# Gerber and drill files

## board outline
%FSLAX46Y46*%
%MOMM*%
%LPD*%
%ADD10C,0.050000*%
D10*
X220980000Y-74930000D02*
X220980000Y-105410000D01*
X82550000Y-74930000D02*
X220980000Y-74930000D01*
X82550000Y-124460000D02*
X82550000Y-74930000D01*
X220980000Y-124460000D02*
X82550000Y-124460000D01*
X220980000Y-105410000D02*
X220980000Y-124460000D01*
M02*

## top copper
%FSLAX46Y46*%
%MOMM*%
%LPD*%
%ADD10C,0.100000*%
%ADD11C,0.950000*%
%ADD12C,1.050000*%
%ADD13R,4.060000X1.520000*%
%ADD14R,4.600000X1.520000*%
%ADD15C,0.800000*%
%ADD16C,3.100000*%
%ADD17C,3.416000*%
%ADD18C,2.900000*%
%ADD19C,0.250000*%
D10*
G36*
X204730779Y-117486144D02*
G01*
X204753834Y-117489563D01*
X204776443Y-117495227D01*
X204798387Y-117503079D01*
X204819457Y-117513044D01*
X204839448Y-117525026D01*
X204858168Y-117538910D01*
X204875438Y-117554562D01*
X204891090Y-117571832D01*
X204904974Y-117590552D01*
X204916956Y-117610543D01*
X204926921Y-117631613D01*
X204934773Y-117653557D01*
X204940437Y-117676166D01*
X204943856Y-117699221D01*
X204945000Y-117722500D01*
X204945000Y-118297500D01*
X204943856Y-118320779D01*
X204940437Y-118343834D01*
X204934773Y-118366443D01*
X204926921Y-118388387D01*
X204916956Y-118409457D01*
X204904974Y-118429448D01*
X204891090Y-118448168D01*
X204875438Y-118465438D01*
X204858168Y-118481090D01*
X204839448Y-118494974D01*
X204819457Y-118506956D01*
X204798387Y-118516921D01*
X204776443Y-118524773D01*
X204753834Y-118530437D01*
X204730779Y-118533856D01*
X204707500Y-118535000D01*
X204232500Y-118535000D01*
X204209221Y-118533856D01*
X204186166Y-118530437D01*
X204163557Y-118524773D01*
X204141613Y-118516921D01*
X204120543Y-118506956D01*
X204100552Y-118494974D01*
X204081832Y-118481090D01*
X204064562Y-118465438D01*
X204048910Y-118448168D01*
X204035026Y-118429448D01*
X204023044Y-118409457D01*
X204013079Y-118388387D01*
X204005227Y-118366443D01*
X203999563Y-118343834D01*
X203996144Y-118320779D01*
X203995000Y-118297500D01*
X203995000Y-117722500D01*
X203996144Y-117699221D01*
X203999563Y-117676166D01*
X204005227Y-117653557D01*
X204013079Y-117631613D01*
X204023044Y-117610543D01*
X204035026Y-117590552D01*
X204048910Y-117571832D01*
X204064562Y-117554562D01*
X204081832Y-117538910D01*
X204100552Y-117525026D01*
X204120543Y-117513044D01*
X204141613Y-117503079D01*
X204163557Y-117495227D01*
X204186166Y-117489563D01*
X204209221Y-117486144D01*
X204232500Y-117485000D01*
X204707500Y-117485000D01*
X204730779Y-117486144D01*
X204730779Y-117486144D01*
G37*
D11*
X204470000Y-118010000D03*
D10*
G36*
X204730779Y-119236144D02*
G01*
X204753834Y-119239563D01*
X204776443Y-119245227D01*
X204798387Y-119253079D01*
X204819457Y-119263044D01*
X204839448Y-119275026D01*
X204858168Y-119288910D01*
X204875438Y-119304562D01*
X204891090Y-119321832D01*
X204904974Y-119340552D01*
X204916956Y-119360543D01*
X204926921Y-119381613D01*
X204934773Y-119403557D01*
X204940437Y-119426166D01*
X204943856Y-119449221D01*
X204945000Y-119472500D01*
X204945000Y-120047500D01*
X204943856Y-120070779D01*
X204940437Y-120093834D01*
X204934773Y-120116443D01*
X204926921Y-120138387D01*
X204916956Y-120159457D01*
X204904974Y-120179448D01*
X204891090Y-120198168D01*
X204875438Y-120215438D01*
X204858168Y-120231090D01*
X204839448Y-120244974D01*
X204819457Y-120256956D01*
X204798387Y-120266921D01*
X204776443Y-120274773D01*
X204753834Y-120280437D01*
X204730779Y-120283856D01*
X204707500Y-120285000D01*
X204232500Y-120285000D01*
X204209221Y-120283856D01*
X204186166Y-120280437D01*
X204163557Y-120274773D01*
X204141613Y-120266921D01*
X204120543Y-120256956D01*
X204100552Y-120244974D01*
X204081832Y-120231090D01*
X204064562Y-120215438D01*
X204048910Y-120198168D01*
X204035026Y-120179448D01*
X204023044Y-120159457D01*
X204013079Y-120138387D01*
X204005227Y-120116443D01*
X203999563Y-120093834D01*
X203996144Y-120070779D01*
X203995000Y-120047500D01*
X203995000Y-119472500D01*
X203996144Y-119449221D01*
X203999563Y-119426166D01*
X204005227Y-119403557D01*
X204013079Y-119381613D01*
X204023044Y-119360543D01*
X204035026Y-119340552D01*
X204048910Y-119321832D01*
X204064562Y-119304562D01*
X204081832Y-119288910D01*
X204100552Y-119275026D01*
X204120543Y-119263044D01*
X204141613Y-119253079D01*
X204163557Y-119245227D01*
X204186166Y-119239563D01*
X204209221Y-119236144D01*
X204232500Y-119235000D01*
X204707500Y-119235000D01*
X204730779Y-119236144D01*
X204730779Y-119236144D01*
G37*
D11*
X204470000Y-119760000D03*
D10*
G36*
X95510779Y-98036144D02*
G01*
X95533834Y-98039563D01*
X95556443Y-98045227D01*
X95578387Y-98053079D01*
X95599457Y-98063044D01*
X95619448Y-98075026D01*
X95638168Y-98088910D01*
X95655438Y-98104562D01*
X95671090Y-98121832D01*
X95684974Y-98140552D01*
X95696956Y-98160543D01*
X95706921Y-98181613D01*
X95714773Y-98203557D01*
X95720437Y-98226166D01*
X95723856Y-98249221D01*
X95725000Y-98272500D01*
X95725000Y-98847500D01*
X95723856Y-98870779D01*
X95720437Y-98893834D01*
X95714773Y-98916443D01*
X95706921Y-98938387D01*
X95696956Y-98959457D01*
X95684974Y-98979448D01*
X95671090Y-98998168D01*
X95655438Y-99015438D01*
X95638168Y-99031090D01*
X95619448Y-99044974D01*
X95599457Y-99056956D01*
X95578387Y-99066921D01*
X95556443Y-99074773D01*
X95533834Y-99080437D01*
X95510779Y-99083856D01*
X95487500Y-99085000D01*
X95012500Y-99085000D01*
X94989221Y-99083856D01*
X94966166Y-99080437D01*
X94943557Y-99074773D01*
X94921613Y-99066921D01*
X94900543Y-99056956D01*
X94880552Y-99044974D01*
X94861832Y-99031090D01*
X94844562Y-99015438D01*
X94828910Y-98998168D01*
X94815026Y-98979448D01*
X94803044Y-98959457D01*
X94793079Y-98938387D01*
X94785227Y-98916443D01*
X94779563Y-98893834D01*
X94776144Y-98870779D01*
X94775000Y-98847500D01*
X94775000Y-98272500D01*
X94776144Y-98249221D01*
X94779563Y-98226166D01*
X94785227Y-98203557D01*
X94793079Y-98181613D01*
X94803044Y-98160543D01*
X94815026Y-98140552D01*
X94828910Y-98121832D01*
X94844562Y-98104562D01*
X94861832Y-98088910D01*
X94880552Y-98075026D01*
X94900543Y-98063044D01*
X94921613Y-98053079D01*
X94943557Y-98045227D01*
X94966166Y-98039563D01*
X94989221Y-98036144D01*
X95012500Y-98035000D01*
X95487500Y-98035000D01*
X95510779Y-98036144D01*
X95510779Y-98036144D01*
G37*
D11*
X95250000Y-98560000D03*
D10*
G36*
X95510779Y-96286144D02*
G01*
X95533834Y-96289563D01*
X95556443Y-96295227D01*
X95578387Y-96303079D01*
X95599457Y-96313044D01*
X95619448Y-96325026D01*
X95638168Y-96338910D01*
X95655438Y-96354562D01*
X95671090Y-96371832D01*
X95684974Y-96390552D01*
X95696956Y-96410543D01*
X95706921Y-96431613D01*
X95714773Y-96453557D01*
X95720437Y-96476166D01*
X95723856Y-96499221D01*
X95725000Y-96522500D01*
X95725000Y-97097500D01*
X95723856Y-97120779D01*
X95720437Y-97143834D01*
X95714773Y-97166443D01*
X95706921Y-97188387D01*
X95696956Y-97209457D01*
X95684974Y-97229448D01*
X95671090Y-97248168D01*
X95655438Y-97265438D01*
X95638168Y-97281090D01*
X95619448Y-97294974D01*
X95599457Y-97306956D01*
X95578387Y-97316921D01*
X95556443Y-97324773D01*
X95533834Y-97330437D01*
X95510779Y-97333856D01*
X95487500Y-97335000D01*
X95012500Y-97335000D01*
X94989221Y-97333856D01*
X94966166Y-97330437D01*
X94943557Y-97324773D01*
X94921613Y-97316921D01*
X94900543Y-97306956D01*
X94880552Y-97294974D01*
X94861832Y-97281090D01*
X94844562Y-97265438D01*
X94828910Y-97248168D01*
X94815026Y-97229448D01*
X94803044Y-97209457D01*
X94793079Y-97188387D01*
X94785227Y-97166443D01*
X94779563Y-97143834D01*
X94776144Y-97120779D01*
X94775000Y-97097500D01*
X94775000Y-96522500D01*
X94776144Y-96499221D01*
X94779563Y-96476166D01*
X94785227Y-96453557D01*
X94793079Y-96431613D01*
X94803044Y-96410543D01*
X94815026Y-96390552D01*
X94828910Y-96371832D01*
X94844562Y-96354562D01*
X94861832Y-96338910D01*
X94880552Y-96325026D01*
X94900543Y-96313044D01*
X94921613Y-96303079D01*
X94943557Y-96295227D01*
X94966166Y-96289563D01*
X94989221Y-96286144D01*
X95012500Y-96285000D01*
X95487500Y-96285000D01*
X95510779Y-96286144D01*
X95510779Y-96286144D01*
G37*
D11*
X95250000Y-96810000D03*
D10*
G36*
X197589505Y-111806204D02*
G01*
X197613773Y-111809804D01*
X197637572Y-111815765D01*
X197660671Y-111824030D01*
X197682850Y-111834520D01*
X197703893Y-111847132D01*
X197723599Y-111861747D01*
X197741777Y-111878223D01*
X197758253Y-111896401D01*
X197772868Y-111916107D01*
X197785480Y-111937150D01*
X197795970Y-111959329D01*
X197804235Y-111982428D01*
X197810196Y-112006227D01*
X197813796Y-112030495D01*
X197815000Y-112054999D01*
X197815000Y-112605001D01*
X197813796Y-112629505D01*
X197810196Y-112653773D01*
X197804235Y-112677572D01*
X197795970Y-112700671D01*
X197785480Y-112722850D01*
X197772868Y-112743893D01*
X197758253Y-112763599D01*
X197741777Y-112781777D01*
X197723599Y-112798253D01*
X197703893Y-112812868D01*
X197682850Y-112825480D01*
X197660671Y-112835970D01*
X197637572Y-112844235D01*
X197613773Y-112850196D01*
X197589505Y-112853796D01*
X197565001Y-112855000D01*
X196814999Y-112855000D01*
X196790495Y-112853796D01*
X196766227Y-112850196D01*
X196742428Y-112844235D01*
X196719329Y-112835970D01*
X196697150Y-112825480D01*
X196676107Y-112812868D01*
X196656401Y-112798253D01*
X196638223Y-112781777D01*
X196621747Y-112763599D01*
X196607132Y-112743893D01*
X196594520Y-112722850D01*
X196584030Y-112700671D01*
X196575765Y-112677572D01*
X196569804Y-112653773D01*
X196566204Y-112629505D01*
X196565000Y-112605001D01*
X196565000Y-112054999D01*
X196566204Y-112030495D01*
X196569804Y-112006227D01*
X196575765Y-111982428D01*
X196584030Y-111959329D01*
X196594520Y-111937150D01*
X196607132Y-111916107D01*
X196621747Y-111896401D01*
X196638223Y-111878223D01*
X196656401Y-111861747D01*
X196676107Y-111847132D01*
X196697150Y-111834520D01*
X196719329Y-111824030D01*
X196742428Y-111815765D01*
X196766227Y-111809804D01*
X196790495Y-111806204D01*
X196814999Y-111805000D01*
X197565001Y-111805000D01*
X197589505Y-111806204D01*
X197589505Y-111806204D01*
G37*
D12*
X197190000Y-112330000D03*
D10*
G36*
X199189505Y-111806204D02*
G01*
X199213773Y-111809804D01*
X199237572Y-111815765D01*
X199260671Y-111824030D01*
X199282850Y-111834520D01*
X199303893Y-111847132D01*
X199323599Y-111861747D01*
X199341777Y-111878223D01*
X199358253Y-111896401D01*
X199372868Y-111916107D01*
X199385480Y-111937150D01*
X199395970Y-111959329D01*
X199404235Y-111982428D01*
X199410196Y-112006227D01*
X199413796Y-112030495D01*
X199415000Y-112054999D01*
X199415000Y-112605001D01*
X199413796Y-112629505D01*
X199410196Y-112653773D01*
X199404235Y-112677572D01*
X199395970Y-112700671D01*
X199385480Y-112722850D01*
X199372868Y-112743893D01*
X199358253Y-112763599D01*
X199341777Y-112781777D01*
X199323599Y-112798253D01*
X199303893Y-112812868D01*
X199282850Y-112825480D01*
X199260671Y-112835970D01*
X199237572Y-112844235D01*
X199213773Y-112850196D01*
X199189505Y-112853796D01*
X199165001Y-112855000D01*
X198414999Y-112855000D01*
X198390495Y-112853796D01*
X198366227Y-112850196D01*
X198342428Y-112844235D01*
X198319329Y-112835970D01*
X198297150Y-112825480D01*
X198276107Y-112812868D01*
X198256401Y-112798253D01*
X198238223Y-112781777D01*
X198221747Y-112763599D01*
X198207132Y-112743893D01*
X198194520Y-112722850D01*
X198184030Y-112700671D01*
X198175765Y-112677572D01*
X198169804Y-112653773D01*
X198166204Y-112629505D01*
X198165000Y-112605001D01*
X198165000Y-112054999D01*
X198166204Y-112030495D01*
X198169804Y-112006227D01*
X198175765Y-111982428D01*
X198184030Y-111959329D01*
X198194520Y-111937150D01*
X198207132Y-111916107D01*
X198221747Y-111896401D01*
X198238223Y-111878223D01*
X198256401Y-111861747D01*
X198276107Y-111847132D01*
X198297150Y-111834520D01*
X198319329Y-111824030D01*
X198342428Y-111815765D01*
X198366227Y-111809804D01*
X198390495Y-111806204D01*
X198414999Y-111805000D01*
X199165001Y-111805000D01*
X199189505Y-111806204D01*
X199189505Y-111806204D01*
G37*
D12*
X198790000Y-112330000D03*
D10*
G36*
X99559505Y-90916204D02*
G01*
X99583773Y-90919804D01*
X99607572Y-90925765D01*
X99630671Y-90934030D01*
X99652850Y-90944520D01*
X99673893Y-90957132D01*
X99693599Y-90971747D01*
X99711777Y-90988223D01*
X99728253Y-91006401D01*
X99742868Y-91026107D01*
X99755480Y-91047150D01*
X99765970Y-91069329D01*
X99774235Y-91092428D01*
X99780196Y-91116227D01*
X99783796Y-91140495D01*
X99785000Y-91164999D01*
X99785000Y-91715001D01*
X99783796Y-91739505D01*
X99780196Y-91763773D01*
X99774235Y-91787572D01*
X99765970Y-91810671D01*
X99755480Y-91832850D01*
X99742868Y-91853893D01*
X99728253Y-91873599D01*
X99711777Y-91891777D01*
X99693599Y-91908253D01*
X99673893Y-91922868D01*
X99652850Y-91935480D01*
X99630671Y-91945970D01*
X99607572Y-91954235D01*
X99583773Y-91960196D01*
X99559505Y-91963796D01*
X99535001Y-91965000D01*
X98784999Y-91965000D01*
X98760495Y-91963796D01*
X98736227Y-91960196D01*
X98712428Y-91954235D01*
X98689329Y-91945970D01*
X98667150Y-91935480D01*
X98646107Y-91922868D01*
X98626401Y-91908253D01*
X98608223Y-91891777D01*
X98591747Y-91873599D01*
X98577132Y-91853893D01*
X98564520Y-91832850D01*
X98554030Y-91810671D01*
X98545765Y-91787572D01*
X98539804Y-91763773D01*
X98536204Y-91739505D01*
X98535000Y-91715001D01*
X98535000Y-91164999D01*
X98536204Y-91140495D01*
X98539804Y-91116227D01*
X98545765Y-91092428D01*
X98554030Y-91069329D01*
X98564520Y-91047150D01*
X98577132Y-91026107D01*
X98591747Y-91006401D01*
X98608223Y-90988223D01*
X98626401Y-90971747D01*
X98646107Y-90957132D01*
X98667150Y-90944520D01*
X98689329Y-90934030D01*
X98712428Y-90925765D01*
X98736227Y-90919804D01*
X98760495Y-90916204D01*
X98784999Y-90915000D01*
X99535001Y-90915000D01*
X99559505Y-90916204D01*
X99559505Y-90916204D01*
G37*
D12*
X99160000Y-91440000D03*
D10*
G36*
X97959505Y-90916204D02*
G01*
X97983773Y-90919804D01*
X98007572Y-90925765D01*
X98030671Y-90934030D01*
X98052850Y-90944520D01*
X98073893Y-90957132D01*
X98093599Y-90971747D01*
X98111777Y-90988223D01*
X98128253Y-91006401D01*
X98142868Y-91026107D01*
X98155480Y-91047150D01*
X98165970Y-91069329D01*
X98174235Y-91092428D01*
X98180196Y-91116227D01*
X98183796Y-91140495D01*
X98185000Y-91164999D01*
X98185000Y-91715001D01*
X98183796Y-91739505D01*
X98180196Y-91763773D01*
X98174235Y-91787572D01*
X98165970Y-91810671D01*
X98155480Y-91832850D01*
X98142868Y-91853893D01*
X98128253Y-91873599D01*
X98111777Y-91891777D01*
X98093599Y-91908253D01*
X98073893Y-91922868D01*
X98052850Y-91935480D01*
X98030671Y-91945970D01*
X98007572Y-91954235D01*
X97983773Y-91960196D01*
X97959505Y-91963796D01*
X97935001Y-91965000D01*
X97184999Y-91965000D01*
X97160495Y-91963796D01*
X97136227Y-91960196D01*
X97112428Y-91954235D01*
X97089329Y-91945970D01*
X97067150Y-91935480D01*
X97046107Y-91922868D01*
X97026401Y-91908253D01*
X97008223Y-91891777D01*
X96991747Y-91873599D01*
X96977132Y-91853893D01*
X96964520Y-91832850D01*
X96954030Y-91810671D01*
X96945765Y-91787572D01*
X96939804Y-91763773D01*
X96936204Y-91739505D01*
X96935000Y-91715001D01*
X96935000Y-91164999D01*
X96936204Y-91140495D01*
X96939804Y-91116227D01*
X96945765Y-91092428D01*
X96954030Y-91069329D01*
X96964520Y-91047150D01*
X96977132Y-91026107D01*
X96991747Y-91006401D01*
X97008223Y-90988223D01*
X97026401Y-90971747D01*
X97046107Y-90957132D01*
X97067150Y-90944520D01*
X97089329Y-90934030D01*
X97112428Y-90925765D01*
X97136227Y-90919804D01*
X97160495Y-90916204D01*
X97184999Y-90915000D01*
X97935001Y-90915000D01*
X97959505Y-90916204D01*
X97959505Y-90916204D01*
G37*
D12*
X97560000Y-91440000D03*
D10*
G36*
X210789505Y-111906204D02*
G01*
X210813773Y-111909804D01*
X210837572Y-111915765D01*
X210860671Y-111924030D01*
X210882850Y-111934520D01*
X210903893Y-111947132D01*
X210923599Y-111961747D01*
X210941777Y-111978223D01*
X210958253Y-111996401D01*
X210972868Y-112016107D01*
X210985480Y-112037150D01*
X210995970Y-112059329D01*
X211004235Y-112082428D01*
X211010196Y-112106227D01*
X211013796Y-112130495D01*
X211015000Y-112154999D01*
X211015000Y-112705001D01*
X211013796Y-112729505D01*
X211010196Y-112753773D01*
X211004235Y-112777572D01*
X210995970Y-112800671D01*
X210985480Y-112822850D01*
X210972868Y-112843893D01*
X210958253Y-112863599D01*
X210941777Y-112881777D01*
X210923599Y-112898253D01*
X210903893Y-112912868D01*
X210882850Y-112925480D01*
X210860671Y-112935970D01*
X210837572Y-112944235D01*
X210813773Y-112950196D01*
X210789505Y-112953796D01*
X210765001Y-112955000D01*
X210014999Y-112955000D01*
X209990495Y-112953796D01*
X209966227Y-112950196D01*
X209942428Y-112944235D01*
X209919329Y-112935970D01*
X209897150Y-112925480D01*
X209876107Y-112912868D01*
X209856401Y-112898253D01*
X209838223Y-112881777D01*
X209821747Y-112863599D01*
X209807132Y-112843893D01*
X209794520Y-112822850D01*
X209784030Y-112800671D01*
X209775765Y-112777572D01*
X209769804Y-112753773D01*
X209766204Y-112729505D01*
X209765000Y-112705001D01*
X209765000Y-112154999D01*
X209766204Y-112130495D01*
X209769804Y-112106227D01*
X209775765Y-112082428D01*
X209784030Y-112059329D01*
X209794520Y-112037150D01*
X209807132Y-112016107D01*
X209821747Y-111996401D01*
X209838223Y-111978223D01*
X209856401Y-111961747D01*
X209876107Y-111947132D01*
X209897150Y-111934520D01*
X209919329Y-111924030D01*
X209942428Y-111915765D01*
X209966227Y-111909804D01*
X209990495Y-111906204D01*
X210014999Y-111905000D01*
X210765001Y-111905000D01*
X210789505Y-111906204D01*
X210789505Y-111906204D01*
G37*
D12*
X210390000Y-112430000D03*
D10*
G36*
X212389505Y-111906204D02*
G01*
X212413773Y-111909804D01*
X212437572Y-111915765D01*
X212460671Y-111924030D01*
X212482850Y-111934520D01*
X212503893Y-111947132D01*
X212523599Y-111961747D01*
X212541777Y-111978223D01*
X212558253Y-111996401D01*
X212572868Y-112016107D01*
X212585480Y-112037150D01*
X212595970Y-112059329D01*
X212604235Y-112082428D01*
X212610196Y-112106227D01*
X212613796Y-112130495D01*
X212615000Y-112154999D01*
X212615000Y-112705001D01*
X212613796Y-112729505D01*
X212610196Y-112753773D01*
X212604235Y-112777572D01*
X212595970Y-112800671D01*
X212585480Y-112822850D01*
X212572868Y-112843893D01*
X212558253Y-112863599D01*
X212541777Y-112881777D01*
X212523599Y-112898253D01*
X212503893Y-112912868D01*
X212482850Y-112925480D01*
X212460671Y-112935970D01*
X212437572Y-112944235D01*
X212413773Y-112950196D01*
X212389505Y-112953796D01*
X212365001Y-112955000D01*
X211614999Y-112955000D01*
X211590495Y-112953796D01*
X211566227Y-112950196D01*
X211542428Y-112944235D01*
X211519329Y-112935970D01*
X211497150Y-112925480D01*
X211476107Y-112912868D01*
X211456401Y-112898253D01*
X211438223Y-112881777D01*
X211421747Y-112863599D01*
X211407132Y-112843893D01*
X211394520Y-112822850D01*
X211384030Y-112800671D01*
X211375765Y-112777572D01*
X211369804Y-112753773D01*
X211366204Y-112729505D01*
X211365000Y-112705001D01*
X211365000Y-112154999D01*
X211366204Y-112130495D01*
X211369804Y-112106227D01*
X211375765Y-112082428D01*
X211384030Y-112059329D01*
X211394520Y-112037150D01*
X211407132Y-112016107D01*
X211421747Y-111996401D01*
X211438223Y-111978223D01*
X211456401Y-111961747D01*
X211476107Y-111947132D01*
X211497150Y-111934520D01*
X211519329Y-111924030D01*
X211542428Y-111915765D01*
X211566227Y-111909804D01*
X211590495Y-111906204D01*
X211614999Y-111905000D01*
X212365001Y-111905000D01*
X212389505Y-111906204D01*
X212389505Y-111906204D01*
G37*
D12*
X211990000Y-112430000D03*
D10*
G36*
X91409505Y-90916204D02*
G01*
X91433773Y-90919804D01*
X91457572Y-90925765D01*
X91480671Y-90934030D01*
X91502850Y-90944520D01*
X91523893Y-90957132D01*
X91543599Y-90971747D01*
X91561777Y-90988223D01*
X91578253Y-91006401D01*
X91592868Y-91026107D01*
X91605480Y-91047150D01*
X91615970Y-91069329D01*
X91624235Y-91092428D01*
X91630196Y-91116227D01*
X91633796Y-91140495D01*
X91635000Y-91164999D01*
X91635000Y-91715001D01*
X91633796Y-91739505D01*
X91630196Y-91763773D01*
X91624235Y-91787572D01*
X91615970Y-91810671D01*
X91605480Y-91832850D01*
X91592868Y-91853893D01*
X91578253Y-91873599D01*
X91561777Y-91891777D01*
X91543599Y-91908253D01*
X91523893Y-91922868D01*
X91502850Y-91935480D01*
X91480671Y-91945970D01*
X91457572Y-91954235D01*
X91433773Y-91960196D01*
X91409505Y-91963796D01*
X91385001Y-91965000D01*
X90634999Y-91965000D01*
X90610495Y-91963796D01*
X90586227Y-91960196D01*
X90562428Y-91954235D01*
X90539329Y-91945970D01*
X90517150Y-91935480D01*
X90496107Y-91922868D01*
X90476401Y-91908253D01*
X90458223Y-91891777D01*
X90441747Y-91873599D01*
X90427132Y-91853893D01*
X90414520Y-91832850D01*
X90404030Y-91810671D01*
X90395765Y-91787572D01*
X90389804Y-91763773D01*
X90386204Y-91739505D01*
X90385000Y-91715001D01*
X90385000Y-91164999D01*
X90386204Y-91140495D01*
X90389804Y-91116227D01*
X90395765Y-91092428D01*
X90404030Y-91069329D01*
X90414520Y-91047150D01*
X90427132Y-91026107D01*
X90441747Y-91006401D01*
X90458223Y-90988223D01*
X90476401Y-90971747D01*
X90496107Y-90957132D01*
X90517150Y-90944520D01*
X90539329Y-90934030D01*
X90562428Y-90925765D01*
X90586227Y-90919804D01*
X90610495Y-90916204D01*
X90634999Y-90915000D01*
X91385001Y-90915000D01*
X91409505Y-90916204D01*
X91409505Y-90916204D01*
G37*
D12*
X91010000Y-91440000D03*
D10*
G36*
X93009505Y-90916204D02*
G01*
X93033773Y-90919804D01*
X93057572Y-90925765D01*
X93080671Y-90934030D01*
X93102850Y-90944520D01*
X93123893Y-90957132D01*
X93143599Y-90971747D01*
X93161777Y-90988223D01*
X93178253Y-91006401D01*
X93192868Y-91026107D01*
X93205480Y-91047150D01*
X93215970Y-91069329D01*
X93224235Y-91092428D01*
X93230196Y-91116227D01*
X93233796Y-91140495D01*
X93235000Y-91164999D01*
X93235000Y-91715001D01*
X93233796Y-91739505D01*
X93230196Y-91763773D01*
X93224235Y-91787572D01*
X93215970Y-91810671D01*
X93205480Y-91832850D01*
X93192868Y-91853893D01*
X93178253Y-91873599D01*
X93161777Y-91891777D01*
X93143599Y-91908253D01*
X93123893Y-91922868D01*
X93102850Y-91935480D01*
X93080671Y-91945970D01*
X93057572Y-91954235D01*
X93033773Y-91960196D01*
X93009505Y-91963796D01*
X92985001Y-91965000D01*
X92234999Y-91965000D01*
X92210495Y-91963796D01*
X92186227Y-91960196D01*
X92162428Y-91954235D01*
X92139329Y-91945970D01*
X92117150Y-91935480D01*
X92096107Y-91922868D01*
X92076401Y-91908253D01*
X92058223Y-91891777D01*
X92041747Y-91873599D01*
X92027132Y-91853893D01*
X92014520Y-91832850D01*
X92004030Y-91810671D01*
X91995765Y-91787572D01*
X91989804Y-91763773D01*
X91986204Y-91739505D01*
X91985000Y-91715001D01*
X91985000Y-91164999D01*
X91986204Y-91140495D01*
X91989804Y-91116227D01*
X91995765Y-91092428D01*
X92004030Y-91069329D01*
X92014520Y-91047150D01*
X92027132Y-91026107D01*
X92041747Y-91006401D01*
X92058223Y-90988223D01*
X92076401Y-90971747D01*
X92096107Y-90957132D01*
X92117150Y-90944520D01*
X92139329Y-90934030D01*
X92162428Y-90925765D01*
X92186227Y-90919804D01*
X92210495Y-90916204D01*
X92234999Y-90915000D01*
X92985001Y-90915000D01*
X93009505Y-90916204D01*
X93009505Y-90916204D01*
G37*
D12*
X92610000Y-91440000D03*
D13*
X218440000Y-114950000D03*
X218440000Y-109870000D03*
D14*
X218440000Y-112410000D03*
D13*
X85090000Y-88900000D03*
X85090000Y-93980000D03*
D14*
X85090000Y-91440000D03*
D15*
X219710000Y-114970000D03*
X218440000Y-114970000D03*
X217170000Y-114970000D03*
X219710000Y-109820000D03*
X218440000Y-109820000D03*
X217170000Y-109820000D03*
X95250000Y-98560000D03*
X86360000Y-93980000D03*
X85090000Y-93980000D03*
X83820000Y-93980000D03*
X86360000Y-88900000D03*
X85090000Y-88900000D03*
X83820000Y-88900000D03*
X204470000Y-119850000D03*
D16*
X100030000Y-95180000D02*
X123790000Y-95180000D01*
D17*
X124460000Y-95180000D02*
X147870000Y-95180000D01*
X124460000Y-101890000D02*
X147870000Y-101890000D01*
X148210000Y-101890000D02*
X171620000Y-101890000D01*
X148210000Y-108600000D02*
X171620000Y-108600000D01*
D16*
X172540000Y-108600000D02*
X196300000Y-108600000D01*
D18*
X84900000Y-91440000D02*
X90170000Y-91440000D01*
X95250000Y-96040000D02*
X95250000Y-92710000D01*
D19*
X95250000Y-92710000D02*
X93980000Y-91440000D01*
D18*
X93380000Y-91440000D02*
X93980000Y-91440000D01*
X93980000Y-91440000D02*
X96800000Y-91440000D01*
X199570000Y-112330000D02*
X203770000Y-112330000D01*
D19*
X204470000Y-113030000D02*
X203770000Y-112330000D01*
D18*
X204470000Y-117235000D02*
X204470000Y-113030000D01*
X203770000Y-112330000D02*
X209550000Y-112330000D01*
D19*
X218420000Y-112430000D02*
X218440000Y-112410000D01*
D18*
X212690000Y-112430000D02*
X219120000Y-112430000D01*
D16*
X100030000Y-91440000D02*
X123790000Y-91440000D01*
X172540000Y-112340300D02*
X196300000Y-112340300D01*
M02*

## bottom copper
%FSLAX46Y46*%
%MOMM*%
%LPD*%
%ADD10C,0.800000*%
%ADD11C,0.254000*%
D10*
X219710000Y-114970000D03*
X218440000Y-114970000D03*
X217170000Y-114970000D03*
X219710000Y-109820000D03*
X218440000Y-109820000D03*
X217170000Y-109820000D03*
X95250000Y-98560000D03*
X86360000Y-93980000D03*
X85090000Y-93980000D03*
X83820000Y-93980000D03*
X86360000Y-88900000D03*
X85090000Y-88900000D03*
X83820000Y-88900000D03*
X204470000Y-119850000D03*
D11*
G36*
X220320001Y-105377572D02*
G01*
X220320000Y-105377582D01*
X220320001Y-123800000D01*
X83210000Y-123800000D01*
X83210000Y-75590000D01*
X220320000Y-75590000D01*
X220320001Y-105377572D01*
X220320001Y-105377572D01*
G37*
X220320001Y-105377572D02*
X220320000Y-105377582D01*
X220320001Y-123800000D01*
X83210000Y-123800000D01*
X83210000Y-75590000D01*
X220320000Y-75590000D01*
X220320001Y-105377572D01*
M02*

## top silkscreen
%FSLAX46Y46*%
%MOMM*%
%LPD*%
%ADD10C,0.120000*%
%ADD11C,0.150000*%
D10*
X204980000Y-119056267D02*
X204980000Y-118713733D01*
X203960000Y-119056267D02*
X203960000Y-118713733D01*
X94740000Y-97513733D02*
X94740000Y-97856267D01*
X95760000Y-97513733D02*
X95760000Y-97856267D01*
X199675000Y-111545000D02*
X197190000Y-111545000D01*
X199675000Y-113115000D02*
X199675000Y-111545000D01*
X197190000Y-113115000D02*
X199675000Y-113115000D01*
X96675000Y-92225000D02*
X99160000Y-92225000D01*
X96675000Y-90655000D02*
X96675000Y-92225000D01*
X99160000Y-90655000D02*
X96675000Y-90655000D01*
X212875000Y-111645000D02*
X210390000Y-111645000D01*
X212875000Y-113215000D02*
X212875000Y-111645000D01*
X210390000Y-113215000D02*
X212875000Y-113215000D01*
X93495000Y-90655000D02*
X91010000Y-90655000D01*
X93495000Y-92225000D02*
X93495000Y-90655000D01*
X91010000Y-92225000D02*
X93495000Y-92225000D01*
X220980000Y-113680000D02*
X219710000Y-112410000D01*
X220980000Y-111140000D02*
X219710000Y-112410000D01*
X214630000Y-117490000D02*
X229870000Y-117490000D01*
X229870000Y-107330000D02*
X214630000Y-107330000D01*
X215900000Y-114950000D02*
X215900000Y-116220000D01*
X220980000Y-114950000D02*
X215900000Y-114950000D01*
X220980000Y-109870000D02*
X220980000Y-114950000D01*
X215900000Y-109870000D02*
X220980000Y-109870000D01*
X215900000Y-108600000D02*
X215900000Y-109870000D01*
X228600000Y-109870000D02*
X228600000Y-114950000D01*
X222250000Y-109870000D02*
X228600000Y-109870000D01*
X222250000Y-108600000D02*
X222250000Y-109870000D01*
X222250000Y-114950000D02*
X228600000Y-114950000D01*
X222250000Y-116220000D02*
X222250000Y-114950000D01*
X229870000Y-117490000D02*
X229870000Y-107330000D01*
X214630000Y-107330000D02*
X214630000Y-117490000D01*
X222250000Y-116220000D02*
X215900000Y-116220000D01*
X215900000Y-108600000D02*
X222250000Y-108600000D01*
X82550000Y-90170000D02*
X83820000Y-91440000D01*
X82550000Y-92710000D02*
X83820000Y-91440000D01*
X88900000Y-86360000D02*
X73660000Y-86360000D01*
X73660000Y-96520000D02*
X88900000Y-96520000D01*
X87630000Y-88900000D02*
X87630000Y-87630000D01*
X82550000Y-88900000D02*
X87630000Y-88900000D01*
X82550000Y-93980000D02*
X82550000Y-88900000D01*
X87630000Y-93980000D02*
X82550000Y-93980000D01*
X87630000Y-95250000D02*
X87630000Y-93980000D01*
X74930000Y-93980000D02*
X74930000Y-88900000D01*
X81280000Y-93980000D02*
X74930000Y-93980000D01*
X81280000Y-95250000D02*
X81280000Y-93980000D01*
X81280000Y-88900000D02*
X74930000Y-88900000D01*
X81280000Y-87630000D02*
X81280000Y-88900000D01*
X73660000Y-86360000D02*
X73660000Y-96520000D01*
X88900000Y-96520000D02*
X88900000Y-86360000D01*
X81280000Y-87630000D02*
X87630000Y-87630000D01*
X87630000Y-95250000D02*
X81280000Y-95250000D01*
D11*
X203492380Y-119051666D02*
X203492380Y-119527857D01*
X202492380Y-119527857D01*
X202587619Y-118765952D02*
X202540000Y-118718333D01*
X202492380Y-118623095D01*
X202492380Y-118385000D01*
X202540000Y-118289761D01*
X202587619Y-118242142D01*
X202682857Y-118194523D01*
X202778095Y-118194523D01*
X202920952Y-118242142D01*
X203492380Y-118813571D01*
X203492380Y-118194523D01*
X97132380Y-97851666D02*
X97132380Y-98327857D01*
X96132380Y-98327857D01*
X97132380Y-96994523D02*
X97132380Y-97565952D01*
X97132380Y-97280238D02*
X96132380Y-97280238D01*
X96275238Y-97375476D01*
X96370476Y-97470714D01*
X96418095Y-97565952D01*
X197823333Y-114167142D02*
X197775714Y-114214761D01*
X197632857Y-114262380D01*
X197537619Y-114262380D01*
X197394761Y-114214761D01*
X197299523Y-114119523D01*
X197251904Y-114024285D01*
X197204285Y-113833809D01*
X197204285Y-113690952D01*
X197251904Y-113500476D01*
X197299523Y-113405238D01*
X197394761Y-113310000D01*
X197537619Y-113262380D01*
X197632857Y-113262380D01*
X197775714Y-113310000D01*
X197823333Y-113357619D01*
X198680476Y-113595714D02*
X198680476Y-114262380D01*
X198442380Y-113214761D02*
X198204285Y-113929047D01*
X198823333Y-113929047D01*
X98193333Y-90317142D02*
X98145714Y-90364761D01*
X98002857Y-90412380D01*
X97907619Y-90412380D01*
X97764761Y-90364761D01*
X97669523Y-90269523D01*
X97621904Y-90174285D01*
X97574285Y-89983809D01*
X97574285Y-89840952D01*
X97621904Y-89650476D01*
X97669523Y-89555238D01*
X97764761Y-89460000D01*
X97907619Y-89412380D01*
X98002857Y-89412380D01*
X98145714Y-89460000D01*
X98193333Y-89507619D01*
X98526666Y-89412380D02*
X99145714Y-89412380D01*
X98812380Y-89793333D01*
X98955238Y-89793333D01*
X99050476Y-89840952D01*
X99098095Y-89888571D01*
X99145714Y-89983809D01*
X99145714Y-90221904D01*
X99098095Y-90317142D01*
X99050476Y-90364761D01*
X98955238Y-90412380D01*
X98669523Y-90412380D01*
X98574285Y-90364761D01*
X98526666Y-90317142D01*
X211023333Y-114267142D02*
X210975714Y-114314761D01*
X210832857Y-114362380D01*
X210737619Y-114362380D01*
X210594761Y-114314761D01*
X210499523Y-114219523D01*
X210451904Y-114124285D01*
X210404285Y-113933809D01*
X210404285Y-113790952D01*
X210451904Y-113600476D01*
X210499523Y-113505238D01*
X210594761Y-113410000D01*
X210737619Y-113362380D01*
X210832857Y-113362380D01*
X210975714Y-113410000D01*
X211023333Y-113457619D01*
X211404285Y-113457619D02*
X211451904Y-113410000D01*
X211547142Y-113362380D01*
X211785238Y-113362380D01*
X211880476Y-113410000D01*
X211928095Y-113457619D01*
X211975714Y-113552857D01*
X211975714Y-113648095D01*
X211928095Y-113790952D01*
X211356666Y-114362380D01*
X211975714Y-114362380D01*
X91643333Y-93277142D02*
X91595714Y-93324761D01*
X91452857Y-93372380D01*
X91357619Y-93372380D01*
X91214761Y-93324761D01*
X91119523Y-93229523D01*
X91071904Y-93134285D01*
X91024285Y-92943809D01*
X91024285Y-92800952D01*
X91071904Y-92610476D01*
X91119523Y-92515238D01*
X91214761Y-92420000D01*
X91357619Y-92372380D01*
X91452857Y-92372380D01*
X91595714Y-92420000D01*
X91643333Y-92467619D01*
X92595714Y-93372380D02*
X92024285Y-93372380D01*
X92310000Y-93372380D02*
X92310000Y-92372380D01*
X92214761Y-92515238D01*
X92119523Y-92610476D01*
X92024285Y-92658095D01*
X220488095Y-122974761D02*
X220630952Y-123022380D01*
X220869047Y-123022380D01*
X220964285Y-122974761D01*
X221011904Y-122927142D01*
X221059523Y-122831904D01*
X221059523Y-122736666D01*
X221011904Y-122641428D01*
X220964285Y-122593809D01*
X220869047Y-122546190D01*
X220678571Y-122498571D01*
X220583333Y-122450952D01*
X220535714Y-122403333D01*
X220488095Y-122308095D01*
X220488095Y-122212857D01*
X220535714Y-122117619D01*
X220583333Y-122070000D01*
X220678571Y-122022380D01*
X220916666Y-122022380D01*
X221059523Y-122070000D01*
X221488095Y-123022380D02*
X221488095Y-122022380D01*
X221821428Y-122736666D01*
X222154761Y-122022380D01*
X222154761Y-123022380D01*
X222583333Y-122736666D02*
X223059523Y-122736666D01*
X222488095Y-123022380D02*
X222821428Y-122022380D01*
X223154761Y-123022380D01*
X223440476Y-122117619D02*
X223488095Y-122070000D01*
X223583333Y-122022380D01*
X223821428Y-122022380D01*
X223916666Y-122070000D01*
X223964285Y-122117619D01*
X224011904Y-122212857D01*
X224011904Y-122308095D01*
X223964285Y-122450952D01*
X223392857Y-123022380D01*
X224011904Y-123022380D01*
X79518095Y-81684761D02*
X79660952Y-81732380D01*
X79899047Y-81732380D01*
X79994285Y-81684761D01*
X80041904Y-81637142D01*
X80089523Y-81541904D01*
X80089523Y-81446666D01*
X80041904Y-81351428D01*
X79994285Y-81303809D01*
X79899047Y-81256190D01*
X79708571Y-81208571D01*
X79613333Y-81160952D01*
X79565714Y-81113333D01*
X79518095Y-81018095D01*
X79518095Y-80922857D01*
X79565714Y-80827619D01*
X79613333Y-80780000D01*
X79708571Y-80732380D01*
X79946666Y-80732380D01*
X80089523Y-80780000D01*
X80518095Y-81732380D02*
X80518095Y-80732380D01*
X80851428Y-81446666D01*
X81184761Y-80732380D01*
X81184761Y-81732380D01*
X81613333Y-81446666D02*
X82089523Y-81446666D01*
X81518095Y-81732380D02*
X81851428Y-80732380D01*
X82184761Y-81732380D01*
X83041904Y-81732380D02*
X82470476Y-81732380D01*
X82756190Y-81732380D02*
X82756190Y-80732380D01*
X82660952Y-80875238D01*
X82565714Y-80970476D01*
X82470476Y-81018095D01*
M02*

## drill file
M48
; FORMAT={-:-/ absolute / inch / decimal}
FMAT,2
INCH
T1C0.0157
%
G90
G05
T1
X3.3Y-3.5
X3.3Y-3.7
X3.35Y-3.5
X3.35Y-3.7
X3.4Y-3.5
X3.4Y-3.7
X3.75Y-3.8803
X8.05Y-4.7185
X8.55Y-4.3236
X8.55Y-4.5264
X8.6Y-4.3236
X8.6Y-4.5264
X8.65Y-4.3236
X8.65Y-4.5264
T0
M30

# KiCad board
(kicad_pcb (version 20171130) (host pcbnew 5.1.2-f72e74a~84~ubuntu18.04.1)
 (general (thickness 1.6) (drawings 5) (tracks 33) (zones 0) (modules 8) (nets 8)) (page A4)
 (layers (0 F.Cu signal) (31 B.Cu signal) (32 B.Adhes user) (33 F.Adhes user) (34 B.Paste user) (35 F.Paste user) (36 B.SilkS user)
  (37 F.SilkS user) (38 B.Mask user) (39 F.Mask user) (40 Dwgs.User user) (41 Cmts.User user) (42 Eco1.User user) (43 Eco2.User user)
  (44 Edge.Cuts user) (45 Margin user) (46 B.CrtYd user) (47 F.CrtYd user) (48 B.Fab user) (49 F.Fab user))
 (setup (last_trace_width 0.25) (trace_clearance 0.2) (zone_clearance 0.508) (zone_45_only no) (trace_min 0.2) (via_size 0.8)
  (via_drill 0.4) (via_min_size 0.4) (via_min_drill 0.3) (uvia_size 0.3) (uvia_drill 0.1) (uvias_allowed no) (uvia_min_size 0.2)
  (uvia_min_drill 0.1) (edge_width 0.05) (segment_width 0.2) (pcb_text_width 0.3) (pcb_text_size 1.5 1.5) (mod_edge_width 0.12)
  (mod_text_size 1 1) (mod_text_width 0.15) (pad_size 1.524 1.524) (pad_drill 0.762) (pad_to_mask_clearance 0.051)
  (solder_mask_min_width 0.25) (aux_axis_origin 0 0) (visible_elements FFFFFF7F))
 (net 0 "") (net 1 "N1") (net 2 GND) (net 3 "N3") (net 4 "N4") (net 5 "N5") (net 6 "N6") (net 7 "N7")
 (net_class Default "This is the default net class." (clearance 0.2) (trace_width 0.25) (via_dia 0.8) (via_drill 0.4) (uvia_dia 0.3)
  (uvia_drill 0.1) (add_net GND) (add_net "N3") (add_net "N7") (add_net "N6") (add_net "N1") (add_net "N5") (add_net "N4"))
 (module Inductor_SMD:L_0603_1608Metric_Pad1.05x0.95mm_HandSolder (layer F.Cu) (at 204.47 118.885 90)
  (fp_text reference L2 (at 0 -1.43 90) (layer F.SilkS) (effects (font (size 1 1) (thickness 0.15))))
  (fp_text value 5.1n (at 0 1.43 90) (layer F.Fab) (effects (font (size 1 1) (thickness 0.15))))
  (fp_line (start -0.171267 0.51) (end 0.171267 0.51) (layer F.SilkS) (width 0.12))
  (fp_line (start -0.171267 -0.51) (end 0.171267 -0.51) (layer F.SilkS) (width 0.12))
  (pad 2 smd roundrect (at 0.875 0 90) (size 1.05 0.95) (layers F.Cu F.Paste F.Mask) (roundrect_rratio 0.25) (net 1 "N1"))
  (pad 1 smd roundrect (at -0.875 0 90) (size 1.05 0.95) (layers F.Cu F.Paste F.Mask) (roundrect_rratio 0.25) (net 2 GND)))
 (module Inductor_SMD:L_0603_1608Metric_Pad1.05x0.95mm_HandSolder (layer F.Cu) (at 95.25 97.685 270)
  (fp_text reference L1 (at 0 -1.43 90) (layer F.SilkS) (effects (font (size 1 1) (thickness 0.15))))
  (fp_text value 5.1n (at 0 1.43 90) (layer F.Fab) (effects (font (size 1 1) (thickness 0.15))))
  (fp_line (start -0.171267 0.51) (end 0.171267 0.51) (layer F.SilkS) (width 0.12))
  (fp_line (start -0.171267 -0.51) (end 0.171267 -0.51) (layer F.SilkS) (width 0.12))
  (pad 2 smd roundrect (at 0.875 0 270) (size 1.05 0.95) (layers F.Cu F.Paste F.Mask) (roundrect_rratio 0.25) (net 2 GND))
  (pad 1 smd roundrect (at -0.875 0 270) (size 1.05 0.95) (layers F.Cu F.Paste F.Mask) (roundrect_rratio 0.25) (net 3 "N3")))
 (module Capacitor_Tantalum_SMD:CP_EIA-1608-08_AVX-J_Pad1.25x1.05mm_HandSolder (layer F.Cu) (at 197.99 112.33 180)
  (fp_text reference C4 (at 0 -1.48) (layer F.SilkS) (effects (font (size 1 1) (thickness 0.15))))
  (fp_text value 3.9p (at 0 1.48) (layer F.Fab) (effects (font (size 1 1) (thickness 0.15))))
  (fp_line (start -1.685 0.785) (end 0.8 0.785) (layer F.SilkS) (width 0.12))
  (fp_line (start -1.685 -0.785) (end -1.685 0.785) (layer F.SilkS) (width 0.12))
  (fp_line (start 0.8 -0.785) (end -1.685 -0.785) (layer F.SilkS) (width 0.12))
  (pad 2 smd roundrect (at 0.8 0 180) (size 1.25 1.05) (layers F.Cu F.Paste F.Mask) (roundrect_rratio 0.238095) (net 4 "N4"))
  (pad 1 smd roundrect (at -0.8 0 180) (size 1.25 1.05) (layers F.Cu F.Paste F.Mask) (roundrect_rratio 0.238095) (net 1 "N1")))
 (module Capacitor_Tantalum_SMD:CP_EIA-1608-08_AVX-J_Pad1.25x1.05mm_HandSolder (layer F.Cu) (at 98.36 91.44)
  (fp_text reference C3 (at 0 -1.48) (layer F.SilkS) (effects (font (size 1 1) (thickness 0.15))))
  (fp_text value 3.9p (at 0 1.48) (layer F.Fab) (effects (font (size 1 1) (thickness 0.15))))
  (fp_line (start -1.685 0.785) (end 0.8 0.785) (layer F.SilkS) (width 0.12))
  (fp_line (start -1.685 -0.785) (end -1.685 0.785) (layer F.SilkS) (width 0.12))
  (fp_line (start 0.8 -0.785) (end -1.685 -0.785) (layer F.SilkS) (width 0.12))
  (pad 2 smd roundrect (at 0.8 0) (size 1.25 1.05) (layers F.Cu F.Paste F.Mask) (roundrect_rratio 0.238095) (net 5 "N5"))
  (pad 1 smd roundrect (at -0.8 0) (size 1.25 1.05) (layers F.Cu F.Paste F.Mask) (roundrect_rratio 0.238095) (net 3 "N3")))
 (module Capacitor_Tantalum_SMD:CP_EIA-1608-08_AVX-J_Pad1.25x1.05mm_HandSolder (layer F.Cu) (at 211.19 112.43 180)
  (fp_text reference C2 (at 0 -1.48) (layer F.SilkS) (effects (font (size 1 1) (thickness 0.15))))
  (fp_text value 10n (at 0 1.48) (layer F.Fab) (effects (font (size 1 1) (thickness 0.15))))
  (fp_line (start -1.685 0.785) (end 0.8 0.785) (layer F.SilkS) (width 0.12))
  (fp_line (start -1.685 -0.785) (end -1.685 0.785) (layer F.SilkS) (width 0.12))
  (fp_line (start 0.8 -0.785) (end -1.685 -0.785) (layer F.SilkS) (width 0.12))
  (pad 2 smd roundrect (at 0.8 0 180) (size 1.25 1.05) (layers F.Cu F.Paste F.Mask) (roundrect_rratio 0.238095) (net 1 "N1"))
  (pad 1 smd roundrect (at -0.8 0 180) (size 1.25 1.05) (layers F.Cu F.Paste F.Mask) (roundrect_rratio 0.238095) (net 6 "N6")))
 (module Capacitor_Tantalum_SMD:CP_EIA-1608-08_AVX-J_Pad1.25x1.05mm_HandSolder (layer F.Cu) (at 91.81 91.44 180)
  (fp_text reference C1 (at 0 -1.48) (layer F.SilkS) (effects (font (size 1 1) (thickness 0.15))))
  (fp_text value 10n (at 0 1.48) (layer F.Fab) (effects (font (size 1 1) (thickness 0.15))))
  (fp_line (start -1.685 0.785) (end 0.8 0.785) (layer F.SilkS) (width 0.12))
  (fp_line (start -1.685 -0.785) (end -1.685 0.785) (layer F.SilkS) (width 0.12))
  (fp_line (start 0.8 -0.785) (end -1.685 -0.785) (layer F.SilkS) (width 0.12))
  (pad 2 smd roundrect (at 0.8 0 180) (size 1.25 1.05) (layers F.Cu F.Paste F.Mask) (roundrect_rratio 0.238095) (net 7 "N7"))
  (pad 1 smd roundrect (at -0.8 0 180) (size 1.25 1.05) (layers F.Cu F.Paste F.Mask) (roundrect_rratio 0.238095) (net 3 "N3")))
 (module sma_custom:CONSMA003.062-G (layer F.Cu) (at 222.25 114.95)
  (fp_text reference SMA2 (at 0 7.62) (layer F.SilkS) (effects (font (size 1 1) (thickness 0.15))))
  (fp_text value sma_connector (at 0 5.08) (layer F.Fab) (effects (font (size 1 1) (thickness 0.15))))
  (fp_line (start -1.27 -1.27) (end -2.54 -2.54) (layer F.SilkS) (width 0.12))
  (fp_line (start -1.27 -3.81) (end -2.54 -2.54) (layer F.SilkS) (width 0.12))
  (fp_line (start -7.62 2.54) (end 7.62 2.54) (layer F.SilkS) (width 0.12))
  (fp_line (start 7.62 -7.62) (end -7.62 -7.62) (layer F.SilkS) (width 0.12))
  (fp_line (start -6.35 0) (end -6.35 1.27) (layer F.SilkS) (width 0.12))
  (fp_line (start -1.27 0) (end -6.35 0) (layer F.SilkS) (width 0.12))
  (fp_line (start -1.27 -5.08) (end -1.27 0) (layer F.SilkS) (width 0.12))
  (fp_line (start -6.35 -5.08) (end -1.27 -5.08) (layer F.SilkS) (width 0.12))
  (fp_line (start -6.35 -6.35) (end -6.35 -5.08) (layer F.SilkS) (width 0.12))
  (fp_line (start 6.35 -5.08) (end 6.35 0) (layer F.SilkS) (width 0.12))
  (fp_line (start 0 -5.08) (end 6.35 -5.08) (layer F.SilkS) (width 0.12))
  (fp_line (start 0 -6.35) (end 0 -5.08) (layer F.SilkS) (width 0.12))
  (fp_line (start 0 0) (end 6.35 0) (layer F.SilkS) (width 0.12))
  (fp_line (start 0 1.27) (end 0 0) (layer F.SilkS) (width 0.12))
  (fp_line (start 7.62 2.54) (end 7.62 -7.62) (layer F.SilkS) (width 0.12))
  (fp_line (start -7.62 -7.62) (end -7.62 2.54) (layer F.SilkS) (width 0.12))
  (fp_line (start 0 1.27) (end -6.35 1.27) (layer F.SilkS) (width 0.12))
  (fp_line (start -6.35 -6.35) (end 0 -6.35) (layer F.SilkS) (width 0.12))
  (pad 3 smd rect (at -3.81 0) (size 4.06 1.52) (layers F.Cu F.Paste F.Mask) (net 2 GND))
  (pad 2 smd rect (at -3.81 -5.08) (size 4.06 1.52) (layers F.Cu F.Paste F.Mask) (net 2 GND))
  (pad 1 smd rect (at -3.81 -2.54) (size 4.6 1.52) (layers F.Cu F.Paste F.Mask) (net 6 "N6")))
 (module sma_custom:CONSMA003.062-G (layer F.Cu) (at 81.28 88.9 180)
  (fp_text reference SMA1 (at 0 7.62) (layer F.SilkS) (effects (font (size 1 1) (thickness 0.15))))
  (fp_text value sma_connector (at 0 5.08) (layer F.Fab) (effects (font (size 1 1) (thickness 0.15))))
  (fp_line (start -1.27 -1.27) (end -2.54 -2.54) (layer F.SilkS) (width 0.12))
  (fp_line (start -1.27 -3.81) (end -2.54 -2.54) (layer F.SilkS) (width 0.12))
  (fp_line (start -7.62 2.54) (end 7.62 2.54) (layer F.SilkS) (width 0.12))
  (fp_line (start 7.62 -7.62) (end -7.62 -7.62) (layer F.SilkS) (width 0.12))
  (fp_line (start -6.35 0) (end -6.35 1.27) (layer F.SilkS) (width 0.12))
  (fp_line (start -1.27 0) (end -6.35 0) (layer F.SilkS) (width 0.12))
  (fp_line (start -1.27 -5.08) (end -1.27 0) (layer F.SilkS) (width 0.12))
  (fp_line (start -6.35 -5.08) (end -1.27 -5.08) (layer F.SilkS) (width 0.12))
  (fp_line (start -6.35 -6.35) (end -6.35 -5.08) (layer F.SilkS) (width 0.12))
  (fp_line (start 6.35 -5.08) (end 6.35 0) (layer F.SilkS) (width 0.12))
  (fp_line (start 0 -5.08) (end 6.35 -5.08) (layer F.SilkS) (width 0.12))
  (fp_line (start 0 -6.35) (end 0 -5.08) (layer F.SilkS) (width 0.12))
  (fp_line (start 0 0) (end 6.35 0) (layer F.SilkS) (width 0.12))
  (fp_line (start 0 1.27) (end 0 0) (layer F.SilkS) (width 0.12))
  (fp_line (start 7.62 2.54) (end 7.62 -7.62) (layer F.SilkS) (width 0.12))
  (fp_line (start -7.62 -7.62) (end -7.62 2.54) (layer F.SilkS) (width 0.12))
  (fp_line (start 0 1.27) (end -6.35 1.27) (layer F.SilkS) (width 0.12))
  (fp_line (start -6.35 -6.35) (end 0 -6.35) (layer F.SilkS) (width 0.12))
  (pad 3 smd rect (at -3.81 0 180) (size 4.06 1.52) (layers F.Cu F.Paste F.Mask) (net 2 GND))
  (pad 2 smd rect (at -3.81 -5.08 180) (size 4.06 1.52) (layers F.Cu F.Paste F.Mask) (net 2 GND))
  (pad 1 smd rect (at -3.81 -2.54 180) (size 4.6 1.52) (layers F.Cu F.Paste F.Mask) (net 7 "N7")))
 (gr_line (start 220.98 74.93) (end 220.98 105.41) (layer Edge.Cuts) (width 0.05))
 (gr_line (start 82.55 74.93) (end 220.98 74.93) (layer Edge.Cuts) (width 0.05))
 (gr_line (start 82.55 124.46) (end 82.55 74.93) (layer Edge.Cuts) (width 0.05))
 (gr_line (start 220.98 124.46) (end 82.55 124.46) (layer Edge.Cuts) (width 0.05))
 (gr_line (start 220.98 105.41) (end 220.98 124.46) (layer Edge.Cuts) (width 0.05))
 (segment (start 100.03 95.18) (end 123.79 95.18) (width 3.1) (layer F.Cu) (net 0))
 (segment (start 124.46 95.18) (end 147.87 95.18) (width 3.416) (layer F.Cu) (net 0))
 (segment (start 124.46 101.89) (end 147.87 101.89) (width 3.416) (layer F.Cu) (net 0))
 (segment (start 148.21 101.89) (end 171.62 101.89) (width 3.416) (layer F.Cu) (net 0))
 (segment (start 148.21 108.6) (end 171.62 108.6) (width 3.416) (layer F.Cu) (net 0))
 (segment (start 172.54 108.6) (end 196.3 108.6) (width 3.1) (layer F.Cu) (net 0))
 (via (at 219.71 114.97) (size 0.8) (drill 0.4) (layers F.Cu B.Cu) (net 2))
 (via (at 218.44 114.97) (size 0.8) (drill 0.4) (layers F.Cu B.Cu) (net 2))
 (via (at 217.17 114.97) (size 0.8) (drill 0.4) (layers F.Cu B.Cu) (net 2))
 (via (at 219.71 109.82) (size 0.8) (drill 0.4) (layers F.Cu B.Cu) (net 2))
 (via (at 218.44 109.82) (size 0.8) (drill 0.4) (layers F.Cu B.Cu) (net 2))
 (via (at 217.17 109.82) (size 0.8) (drill 0.4) (layers F.Cu B.Cu) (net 2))
 (via (at 95.25 98.56) (size 0.8) (drill 0.4) (layers F.Cu B.Cu) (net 2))
 (via (at 86.36 93.98) (size 0.8) (drill 0.4) (layers F.Cu B.Cu) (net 2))
 (via (at 85.09 93.98) (size 0.8) (drill 0.4) (layers F.Cu B.Cu) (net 2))
 (via (at 83.82 93.98) (size 0.8) (drill 0.4) (layers F.Cu B.Cu) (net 2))
 (via (at 86.36 88.9) (size 0.8) (drill 0.4) (layers F.Cu B.Cu) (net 2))
 (via (at 85.09 88.9) (size 0.8) (drill 0.4) (layers F.Cu B.Cu) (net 2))
 (via (at 83.82 88.9) (size 0.8) (drill 0.4) (layers F.Cu B.Cu) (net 2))
 (via (at 204.47 119.85) (size 0.8) (drill 0.4) (layers F.Cu B.Cu) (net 2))
 (segment (start 84.9 91.44) (end 90.17 91.44) (width 2.9) (layer F.Cu) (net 7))
 (segment (start 95.25 96.04) (end 95.25 92.71) (width 2.9) (layer F.Cu) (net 3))
 (segment (start 95.25 92.71) (end 93.98 91.44) (width 0.25) (layer F.Cu) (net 3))
 (segment (start 93.38 91.44) (end 93.98 91.44) (width 2.9) (layer F.Cu) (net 3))
 (segment (start 93.98 91.44) (end 96.8 91.44) (width 2.9) (layer F.Cu) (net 3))
 (segment (start 199.57 112.33) (end 203.77 112.33) (width 2.9) (layer F.Cu) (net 1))
 (segment (start 204.47 113.03) (end 203.77 112.33) (width 0.25) (layer F.Cu) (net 1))
 (segment (start 204.47 117.235) (end 204.47 113.03) (width 2.9) (layer F.Cu) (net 1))
 (segment (start 203.77 112.33) (end 209.55 112.33) (width 2.9) (layer F.Cu) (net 1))
 (segment (start 218.42 112.43) (end 218.44 112.41) (width 0.25) (layer F.Cu) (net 6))
 (segment (start 212.69 112.43) (end 219.12 112.43) (width 2.9) (layer F.Cu) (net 6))
 (segment (start 100.03 91.44) (end 123.79 91.44) (width 3.1) (layer F.Cu) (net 5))
 (segment (start 172.54 112.3403) (end 196.3 112.3403) (width 3.1) (layer F.Cu) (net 4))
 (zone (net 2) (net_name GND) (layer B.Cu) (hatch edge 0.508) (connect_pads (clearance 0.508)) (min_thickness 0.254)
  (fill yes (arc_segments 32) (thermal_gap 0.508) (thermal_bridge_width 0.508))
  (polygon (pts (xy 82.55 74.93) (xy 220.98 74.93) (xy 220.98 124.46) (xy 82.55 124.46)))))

